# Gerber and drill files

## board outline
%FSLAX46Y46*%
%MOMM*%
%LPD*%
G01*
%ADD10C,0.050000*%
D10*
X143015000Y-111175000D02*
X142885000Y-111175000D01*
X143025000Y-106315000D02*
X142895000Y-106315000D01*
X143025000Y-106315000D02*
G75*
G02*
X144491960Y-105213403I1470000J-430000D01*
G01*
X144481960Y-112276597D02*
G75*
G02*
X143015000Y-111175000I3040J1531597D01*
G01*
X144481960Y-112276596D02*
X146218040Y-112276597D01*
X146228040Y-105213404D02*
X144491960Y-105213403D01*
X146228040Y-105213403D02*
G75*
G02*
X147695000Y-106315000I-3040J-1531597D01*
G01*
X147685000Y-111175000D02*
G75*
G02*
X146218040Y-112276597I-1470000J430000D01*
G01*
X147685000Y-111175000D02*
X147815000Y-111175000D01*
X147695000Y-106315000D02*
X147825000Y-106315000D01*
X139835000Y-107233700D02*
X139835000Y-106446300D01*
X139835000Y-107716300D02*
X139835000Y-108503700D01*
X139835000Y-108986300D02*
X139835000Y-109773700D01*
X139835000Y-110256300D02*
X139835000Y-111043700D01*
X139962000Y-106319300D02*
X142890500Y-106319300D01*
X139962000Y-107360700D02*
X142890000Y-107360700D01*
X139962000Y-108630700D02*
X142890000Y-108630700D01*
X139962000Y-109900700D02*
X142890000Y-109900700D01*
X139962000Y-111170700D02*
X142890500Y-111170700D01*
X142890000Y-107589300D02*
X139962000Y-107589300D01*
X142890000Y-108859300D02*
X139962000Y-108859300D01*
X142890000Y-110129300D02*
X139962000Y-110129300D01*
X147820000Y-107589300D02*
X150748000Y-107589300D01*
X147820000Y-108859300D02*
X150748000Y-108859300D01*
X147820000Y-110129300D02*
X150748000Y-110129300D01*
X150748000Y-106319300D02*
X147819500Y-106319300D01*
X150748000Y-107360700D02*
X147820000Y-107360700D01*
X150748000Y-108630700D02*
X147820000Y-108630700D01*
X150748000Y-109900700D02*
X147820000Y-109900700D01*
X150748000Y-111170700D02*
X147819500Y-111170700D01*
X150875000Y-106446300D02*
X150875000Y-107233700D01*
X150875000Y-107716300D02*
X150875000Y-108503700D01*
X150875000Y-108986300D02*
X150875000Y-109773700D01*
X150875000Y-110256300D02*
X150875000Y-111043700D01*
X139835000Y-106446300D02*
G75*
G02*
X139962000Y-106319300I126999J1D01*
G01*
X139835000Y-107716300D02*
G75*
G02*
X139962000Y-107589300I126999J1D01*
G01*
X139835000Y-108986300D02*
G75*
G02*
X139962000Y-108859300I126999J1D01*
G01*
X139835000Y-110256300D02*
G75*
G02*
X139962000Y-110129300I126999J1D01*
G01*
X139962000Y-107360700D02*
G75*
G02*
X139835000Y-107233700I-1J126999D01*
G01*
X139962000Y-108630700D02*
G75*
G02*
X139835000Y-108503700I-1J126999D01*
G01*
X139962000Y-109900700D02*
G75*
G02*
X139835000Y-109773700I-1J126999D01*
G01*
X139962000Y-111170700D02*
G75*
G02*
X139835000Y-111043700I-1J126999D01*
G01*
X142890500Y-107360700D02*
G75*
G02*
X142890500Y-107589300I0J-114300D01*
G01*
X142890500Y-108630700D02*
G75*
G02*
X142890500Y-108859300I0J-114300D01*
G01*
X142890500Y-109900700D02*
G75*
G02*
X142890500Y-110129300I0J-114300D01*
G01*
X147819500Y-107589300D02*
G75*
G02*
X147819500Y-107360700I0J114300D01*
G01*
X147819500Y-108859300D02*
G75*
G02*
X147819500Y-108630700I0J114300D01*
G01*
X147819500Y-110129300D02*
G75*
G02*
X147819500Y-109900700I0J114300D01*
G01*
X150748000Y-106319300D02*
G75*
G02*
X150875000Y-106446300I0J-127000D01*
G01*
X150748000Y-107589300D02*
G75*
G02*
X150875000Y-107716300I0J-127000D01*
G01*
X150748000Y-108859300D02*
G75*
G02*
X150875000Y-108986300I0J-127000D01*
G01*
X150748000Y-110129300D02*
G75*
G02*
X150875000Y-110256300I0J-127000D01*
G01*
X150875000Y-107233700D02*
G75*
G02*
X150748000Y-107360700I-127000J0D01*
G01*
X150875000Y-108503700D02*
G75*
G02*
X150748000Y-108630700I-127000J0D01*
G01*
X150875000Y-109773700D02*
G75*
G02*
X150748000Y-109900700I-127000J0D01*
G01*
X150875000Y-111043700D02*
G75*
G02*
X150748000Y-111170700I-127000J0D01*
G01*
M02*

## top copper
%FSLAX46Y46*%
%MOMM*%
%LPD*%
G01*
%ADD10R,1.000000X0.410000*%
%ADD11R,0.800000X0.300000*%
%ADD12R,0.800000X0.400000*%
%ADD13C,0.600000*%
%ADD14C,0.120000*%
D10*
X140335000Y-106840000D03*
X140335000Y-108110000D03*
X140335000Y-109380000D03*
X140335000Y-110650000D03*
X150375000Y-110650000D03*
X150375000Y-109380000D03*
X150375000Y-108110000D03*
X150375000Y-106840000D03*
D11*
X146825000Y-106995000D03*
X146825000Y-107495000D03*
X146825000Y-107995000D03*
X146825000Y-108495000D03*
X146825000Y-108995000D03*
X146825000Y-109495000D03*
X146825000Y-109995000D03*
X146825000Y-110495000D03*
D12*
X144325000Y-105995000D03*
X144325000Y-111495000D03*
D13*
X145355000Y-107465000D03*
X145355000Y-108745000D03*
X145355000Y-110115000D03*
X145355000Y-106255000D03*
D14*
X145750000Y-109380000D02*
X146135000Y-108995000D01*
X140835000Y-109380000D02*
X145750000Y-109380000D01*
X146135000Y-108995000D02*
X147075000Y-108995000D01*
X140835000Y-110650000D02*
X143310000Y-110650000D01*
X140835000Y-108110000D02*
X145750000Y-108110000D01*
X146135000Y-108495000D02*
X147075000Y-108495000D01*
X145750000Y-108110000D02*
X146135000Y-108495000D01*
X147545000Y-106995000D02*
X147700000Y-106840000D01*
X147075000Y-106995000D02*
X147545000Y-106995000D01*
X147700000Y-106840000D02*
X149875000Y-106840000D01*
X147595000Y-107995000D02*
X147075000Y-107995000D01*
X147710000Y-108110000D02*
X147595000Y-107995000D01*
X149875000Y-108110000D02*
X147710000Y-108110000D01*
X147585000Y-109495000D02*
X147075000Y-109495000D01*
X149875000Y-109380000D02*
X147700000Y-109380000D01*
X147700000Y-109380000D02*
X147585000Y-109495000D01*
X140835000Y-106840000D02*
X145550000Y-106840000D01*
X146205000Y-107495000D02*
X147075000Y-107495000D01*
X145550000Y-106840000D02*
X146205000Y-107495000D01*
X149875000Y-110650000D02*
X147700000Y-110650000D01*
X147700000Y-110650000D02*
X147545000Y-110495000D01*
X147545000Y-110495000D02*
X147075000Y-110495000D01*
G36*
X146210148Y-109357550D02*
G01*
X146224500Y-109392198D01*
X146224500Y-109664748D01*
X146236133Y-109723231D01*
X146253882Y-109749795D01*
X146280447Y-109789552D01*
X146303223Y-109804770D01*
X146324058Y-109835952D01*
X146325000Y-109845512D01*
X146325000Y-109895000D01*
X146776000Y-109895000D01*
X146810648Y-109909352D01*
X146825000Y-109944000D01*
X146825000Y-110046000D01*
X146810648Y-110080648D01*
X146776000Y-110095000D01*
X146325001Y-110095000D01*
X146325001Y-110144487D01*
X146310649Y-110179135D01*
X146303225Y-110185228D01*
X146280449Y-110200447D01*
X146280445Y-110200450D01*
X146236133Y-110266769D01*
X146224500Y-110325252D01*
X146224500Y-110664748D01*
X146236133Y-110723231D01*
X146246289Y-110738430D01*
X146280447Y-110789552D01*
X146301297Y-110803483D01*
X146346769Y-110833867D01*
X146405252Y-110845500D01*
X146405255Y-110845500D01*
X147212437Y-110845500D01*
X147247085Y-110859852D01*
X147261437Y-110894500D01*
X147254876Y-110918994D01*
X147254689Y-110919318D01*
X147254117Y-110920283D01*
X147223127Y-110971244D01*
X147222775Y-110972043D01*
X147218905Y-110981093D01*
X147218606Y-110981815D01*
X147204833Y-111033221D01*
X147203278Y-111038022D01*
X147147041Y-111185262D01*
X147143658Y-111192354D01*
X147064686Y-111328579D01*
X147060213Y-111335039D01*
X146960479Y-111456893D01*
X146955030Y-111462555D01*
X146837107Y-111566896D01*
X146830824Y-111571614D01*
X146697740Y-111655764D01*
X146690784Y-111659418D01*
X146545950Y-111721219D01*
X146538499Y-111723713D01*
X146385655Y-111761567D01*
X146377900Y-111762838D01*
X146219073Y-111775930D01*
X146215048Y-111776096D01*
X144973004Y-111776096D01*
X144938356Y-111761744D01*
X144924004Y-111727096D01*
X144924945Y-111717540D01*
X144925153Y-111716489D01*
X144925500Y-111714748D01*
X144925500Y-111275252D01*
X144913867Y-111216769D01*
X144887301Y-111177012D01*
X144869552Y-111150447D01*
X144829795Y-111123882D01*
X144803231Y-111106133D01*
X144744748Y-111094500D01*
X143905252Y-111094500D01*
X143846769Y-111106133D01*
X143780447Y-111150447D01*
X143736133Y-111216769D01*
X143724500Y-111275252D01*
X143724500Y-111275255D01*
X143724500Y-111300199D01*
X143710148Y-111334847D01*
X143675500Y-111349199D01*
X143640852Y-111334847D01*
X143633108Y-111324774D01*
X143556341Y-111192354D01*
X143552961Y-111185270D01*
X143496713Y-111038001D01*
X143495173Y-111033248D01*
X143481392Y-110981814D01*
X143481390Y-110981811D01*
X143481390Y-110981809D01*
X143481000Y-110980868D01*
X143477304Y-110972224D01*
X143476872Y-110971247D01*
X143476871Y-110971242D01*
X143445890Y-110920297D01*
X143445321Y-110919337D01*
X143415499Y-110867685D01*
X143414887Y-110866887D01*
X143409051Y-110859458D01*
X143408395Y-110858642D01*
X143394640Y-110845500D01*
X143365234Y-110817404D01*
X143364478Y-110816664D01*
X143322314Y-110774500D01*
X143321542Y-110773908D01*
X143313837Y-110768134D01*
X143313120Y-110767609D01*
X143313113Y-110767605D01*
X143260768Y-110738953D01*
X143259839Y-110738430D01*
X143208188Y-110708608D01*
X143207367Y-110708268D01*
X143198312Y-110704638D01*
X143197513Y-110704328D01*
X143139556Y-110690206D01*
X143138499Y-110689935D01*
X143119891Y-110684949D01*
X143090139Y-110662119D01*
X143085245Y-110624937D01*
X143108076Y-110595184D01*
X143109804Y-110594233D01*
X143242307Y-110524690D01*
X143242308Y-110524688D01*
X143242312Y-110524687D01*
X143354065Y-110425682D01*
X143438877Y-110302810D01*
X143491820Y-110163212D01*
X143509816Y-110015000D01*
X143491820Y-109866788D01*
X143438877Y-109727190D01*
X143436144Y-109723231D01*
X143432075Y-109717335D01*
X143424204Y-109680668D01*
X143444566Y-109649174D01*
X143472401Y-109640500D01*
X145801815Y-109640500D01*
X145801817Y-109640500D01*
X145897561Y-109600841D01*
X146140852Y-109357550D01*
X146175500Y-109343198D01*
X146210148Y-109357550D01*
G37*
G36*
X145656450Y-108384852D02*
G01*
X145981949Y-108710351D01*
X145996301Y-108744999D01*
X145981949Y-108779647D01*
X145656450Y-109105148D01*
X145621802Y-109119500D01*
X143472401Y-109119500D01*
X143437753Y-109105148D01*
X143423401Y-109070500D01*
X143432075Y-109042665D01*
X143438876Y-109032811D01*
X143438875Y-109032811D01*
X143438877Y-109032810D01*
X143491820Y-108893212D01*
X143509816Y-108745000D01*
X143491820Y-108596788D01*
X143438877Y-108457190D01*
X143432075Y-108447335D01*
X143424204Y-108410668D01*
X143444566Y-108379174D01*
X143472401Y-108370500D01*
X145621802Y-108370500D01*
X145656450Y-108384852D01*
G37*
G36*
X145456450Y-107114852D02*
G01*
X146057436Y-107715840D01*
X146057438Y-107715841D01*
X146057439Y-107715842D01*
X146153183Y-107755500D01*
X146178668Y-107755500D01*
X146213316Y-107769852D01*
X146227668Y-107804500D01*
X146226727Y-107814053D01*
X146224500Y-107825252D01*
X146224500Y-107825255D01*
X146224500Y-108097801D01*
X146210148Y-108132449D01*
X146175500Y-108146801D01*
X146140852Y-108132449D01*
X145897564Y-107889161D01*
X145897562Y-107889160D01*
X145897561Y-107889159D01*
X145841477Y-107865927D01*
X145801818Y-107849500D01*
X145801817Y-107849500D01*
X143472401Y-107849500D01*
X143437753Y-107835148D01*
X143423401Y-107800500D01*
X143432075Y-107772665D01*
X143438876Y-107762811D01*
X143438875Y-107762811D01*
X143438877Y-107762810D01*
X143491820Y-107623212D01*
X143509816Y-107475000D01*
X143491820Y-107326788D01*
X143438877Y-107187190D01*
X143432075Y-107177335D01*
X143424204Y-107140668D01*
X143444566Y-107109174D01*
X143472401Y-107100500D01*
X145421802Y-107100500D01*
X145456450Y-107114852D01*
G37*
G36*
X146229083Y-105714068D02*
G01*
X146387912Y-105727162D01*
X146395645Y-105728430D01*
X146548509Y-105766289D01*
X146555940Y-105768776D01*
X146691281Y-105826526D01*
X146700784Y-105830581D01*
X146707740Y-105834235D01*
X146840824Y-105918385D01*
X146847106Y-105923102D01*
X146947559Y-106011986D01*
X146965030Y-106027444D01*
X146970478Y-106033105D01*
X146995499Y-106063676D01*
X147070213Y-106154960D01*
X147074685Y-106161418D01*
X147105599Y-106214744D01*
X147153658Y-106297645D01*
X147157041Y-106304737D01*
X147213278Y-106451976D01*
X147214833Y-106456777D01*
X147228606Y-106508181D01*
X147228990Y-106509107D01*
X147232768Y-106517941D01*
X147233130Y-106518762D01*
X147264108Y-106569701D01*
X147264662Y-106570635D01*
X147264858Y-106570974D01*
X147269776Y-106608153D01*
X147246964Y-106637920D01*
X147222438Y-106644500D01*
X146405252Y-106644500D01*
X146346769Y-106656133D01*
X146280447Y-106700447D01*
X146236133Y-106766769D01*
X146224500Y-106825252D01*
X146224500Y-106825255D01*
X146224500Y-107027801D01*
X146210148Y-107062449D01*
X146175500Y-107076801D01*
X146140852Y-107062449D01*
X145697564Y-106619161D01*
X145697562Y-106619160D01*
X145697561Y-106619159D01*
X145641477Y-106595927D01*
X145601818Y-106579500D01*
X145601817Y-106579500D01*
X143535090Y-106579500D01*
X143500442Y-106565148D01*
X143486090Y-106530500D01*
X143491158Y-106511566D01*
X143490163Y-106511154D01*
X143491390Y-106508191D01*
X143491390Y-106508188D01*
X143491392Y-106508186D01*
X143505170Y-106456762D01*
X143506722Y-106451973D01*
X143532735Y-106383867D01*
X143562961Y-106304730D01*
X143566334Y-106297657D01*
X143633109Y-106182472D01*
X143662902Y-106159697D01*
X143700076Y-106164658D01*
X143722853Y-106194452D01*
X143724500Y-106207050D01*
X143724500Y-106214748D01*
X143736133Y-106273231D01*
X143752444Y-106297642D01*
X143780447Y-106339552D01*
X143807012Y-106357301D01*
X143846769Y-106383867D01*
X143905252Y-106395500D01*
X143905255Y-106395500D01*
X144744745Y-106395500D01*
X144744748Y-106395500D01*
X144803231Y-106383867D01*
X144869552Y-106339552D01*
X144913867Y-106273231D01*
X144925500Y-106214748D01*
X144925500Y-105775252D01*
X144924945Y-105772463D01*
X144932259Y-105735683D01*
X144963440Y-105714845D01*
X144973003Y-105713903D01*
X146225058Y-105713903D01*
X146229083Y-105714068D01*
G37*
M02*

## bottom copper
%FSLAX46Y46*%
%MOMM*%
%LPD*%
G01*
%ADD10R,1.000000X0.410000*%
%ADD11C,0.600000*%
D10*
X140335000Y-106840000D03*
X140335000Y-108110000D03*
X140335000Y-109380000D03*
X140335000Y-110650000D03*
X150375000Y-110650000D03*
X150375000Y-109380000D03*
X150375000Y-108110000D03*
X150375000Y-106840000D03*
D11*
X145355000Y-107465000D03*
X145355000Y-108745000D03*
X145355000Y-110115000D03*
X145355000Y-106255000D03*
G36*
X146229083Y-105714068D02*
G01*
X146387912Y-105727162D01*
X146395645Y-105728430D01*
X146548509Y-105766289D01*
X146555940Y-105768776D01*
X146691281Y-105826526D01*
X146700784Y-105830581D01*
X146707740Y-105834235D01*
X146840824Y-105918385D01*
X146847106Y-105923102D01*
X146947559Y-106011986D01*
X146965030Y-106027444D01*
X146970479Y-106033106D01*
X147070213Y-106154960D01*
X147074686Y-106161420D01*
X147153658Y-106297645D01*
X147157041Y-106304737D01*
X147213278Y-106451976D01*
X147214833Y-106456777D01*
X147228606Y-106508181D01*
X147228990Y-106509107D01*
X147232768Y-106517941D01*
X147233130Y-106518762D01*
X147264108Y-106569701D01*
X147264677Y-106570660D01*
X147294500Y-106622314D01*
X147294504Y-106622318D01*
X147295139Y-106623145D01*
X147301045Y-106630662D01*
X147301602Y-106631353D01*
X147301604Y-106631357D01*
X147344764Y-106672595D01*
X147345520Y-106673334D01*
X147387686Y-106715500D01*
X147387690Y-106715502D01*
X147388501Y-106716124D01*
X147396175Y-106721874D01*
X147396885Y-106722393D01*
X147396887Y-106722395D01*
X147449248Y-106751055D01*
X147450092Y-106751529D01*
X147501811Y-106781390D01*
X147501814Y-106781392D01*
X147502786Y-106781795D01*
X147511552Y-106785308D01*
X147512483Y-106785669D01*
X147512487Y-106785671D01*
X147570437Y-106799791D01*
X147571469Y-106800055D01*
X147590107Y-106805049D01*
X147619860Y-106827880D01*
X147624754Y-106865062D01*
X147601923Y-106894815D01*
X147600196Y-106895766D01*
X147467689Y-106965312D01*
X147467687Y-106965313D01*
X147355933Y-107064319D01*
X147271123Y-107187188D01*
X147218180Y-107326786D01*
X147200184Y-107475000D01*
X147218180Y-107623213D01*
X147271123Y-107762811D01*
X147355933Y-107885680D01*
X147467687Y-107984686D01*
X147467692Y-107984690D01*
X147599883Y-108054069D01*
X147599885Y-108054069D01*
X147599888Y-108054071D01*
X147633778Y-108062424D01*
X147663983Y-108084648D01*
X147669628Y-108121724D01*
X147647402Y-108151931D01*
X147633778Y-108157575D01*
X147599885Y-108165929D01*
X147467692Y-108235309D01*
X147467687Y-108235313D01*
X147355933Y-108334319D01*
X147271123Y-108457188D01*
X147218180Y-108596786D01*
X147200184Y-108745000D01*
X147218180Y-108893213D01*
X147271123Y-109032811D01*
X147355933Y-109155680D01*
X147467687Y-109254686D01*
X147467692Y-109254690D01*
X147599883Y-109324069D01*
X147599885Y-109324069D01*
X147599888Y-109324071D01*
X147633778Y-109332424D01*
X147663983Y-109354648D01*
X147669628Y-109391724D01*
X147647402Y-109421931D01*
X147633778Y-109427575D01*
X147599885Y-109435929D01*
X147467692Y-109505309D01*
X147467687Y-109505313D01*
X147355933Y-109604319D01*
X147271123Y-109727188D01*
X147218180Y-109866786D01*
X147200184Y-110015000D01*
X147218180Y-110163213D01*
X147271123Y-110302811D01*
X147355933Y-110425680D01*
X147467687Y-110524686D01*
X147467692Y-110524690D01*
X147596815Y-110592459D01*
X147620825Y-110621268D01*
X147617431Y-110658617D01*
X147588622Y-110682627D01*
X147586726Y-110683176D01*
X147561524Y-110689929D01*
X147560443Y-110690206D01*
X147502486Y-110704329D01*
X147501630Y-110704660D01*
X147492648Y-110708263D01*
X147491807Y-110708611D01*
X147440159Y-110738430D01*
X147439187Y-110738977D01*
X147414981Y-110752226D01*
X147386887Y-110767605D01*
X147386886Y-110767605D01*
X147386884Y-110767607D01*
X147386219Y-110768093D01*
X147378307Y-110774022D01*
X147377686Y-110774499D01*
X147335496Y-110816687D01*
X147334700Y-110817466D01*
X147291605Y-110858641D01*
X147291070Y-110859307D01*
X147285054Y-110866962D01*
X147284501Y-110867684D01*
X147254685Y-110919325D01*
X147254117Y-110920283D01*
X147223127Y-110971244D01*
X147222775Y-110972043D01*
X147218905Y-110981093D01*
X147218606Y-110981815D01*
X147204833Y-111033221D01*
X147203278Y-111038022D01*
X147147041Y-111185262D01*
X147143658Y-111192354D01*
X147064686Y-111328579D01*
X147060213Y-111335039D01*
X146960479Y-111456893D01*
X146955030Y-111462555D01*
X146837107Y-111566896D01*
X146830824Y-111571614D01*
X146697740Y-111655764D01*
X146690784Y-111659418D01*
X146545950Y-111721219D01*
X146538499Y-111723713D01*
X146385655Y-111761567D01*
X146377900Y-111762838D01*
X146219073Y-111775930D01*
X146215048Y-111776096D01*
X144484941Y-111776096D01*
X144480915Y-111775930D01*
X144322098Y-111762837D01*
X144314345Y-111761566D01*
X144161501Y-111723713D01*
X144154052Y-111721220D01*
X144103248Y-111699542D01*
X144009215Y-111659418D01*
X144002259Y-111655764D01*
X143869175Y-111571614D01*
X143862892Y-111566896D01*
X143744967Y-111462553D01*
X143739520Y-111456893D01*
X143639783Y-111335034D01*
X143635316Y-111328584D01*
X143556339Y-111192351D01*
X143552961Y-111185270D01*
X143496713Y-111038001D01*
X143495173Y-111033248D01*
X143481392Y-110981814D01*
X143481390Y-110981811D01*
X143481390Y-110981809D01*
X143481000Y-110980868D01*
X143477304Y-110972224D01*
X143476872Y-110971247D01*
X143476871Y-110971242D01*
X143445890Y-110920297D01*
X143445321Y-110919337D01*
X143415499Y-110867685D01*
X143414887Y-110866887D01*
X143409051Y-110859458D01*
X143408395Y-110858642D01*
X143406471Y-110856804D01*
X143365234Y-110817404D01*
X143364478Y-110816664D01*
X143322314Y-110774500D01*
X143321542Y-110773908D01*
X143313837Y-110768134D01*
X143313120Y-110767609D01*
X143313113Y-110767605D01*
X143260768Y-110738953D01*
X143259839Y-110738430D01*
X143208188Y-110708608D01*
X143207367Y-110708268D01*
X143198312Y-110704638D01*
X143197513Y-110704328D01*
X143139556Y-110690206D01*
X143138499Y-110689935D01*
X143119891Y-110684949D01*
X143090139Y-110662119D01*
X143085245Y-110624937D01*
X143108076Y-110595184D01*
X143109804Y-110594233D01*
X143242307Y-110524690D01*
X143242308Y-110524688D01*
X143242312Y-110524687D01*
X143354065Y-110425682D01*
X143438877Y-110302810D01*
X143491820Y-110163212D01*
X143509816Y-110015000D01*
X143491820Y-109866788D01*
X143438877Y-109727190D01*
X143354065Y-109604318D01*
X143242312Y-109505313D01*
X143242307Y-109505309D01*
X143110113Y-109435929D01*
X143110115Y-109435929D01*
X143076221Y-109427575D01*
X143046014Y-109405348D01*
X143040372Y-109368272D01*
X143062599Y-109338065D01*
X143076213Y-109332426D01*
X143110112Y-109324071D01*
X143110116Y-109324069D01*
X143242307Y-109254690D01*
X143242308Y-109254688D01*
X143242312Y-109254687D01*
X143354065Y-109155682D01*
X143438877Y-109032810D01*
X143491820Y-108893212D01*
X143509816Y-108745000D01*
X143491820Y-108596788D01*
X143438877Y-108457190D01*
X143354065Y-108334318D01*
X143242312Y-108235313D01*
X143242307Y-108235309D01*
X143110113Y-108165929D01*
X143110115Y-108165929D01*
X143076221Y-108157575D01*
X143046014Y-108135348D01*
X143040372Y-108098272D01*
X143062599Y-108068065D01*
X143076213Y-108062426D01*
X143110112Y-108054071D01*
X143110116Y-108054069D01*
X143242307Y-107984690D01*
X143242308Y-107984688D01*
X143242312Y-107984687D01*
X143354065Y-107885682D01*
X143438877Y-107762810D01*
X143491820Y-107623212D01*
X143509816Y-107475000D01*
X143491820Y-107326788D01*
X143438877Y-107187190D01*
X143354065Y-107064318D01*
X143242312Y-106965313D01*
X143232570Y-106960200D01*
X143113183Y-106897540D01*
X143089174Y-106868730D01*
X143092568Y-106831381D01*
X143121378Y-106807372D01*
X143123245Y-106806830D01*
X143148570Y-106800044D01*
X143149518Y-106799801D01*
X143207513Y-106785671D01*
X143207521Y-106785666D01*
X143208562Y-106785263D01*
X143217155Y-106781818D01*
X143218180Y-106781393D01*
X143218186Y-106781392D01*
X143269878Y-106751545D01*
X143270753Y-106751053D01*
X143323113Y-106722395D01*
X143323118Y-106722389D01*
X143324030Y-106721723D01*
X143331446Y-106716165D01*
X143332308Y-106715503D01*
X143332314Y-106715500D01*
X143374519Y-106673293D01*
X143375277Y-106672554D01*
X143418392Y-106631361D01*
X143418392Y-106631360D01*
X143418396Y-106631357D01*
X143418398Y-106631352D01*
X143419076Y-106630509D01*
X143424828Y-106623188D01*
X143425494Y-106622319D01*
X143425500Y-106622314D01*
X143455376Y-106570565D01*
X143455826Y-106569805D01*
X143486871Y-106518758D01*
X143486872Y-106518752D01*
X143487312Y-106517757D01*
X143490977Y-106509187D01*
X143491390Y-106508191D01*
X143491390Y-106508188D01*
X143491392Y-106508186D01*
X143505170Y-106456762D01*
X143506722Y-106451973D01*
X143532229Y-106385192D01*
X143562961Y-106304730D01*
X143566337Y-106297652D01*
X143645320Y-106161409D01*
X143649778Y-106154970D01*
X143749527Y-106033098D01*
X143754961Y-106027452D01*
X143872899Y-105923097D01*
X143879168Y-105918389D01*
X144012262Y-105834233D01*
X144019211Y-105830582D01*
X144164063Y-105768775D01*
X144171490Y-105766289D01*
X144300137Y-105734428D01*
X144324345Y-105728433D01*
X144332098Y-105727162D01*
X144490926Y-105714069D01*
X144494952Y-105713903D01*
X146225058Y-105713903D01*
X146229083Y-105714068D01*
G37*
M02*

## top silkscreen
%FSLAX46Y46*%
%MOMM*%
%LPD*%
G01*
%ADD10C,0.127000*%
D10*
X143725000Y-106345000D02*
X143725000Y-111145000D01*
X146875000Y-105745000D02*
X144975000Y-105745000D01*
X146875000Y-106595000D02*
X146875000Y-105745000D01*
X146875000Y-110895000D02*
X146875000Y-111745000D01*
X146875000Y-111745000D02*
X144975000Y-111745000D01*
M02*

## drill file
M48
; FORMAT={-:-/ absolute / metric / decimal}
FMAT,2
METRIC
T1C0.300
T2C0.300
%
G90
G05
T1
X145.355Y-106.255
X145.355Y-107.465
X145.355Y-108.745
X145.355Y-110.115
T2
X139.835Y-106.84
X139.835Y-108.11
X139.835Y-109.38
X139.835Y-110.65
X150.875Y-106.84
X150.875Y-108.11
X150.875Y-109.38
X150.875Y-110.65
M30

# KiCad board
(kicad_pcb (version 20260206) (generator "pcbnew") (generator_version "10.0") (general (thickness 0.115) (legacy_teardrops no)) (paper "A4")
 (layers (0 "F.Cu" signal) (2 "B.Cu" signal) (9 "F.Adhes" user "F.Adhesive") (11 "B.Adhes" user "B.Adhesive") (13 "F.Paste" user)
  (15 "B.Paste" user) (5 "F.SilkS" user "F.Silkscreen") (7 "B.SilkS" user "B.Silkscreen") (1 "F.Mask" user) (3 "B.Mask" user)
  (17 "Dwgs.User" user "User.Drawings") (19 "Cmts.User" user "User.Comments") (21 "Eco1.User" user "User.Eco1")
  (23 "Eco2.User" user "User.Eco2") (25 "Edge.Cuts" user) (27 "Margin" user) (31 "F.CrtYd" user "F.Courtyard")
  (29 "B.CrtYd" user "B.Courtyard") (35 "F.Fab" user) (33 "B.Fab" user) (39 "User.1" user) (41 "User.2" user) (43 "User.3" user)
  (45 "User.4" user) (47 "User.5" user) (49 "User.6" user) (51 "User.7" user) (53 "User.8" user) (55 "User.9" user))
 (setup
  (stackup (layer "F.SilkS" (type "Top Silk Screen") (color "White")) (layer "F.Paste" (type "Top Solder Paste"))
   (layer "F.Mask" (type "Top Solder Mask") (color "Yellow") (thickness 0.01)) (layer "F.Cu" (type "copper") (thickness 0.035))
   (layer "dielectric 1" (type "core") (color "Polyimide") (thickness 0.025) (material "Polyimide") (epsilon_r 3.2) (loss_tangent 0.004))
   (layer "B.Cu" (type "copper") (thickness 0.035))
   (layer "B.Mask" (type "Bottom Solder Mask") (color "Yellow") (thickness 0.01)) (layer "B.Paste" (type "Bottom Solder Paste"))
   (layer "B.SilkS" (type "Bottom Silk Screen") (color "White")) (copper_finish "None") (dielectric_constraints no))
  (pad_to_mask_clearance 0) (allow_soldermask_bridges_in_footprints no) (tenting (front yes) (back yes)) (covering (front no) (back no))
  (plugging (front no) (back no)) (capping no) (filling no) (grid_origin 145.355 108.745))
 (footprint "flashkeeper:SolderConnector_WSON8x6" (layer "F.Cu") (at 145.355 108.745)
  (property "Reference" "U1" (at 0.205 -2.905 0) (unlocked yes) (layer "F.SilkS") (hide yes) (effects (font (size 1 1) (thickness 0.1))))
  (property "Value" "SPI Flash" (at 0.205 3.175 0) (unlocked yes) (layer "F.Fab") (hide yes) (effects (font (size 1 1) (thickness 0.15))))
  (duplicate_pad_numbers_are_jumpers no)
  (fp_line (start -5.52 -1.5113) (end -5.52 -2.2987) (stroke (width 0.05) (type default)) (layer "Edge.Cuts"))
  (fp_line (start -5.52 -1.0287) (end -5.52 -0.2413) (stroke (width 0.05) (type default)) (layer "Edge.Cuts"))
  (fp_line (start -5.52 0.2413) (end -5.52 1.0287) (stroke (width 0.05) (type default)) (layer "Edge.Cuts"))
  (fp_line (start -5.52 1.5113) (end -5.52 2.2987) (stroke (width 0.05) (type default)) (layer "Edge.Cuts"))
  (fp_line (start -5.393 -2.4257) (end -2.4645 -2.4257) (stroke (width 0.05) (type default)) (layer "Edge.Cuts"))
  (fp_line (start -5.393 -1.3843) (end -2.465 -1.3843) (stroke (width 0.05) (type default)) (layer "Edge.Cuts"))
  (fp_line (start -5.393 -0.1143) (end -2.465 -0.1143) (stroke (width 0.05) (type default)) (layer "Edge.Cuts"))
  (fp_line (start -5.393 1.1557) (end -2.465 1.1557) (stroke (width 0.05) (type default)) (layer "Edge.Cuts"))
  (fp_line (start -5.393 2.4257) (end -2.4645 2.4257) (stroke (width 0.05) (type default)) (layer "Edge.Cuts"))
  (fp_line (start -2.465 -1.1557) (end -5.393 -1.1557) (stroke (width 0.05) (type default)) (layer "Edge.Cuts"))
  (fp_line (start -2.465 0.1143) (end -5.393 0.1143) (stroke (width 0.05) (type default)) (layer "Edge.Cuts"))
  (fp_line (start -2.465 1.3843) (end -5.393 1.3843) (stroke (width 0.05) (type default)) (layer "Edge.Cuts"))
  (fp_line (start 2.465 -1.1557) (end 5.393 -1.1557) (stroke (width 0.05) (type default)) (layer "Edge.Cuts"))
  (fp_line (start 2.465 0.1143) (end 5.393 0.1143) (stroke (width 0.05) (type default)) (layer "Edge.Cuts"))
  (fp_line (start 2.465 1.3843) (end 5.393 1.3843) (stroke (width 0.05) (type default)) (layer "Edge.Cuts"))
  (fp_line (start 5.393 -2.4257) (end 2.4645 -2.4257) (stroke (width 0.05) (type default)) (layer "Edge.Cuts"))
  (fp_line (start 5.393 -1.3843) (end 2.465 -1.3843) (stroke (width 0.05) (type default)) (layer "Edge.Cuts"))
  (fp_line (start 5.393 -0.1143) (end 2.465 -0.1143) (stroke (width 0.05) (type default)) (layer "Edge.Cuts"))
  (fp_line (start 5.393 1.1557) (end 2.465 1.1557) (stroke (width 0.05) (type default)) (layer "Edge.Cuts"))
  (fp_line (start 5.393 2.4257) (end 2.4645 2.4257) (stroke (width 0.05) (type default)) (layer "Edge.Cuts"))
  (fp_line (start 5.52 -2.2987) (end 5.52 -1.5113) (stroke (width 0.05) (type default)) (layer "Edge.Cuts"))
  (fp_line (start 5.52 -1.0287) (end 5.52 -0.2413) (stroke (width 0.05) (type default)) (layer "Edge.Cuts"))
  (fp_line (start 5.52 0.2413) (end 5.52 1.0287) (stroke (width 0.05) (type default)) (layer "Edge.Cuts"))
  (fp_line (start 5.52 1.5113) (end 5.52 2.2987) (stroke (width 0.05) (type default)) (layer "Edge.Cuts"))
  (fp_arc (start -5.52 -2.2987) (mid -5.482803 -2.388503) (end -5.393 -2.4257) (stroke (width 0.05) (type default)) (layer "Edge.Cuts"))
  (fp_arc (start -5.52 -1.0287) (mid -5.482803 -1.118503) (end -5.393 -1.1557) (stroke (width 0.05) (type default)) (layer "Edge.Cuts"))
  (fp_arc (start -5.52 0.2413) (mid -5.482803 0.151497) (end -5.393 0.1143) (stroke (width 0.05) (type default)) (layer "Edge.Cuts"))
  (fp_arc (start -5.52 1.5113) (mid -5.482803 1.421497) (end -5.393 1.3843) (stroke (width 0.05) (type default)) (layer "Edge.Cuts"))
  (fp_arc (start -5.393 -1.3843) (mid -5.482803 -1.421497) (end -5.52 -1.5113) (stroke (width 0.05) (type default)) (layer "Edge.Cuts"))
  (fp_arc (start -5.393 -0.1143) (mid -5.482803 -0.151497) (end -5.52 -0.2413) (stroke (width 0.05) (type default)) (layer "Edge.Cuts"))
  (fp_arc (start -5.393 1.1557) (mid -5.482803 1.118503) (end -5.52 1.0287) (stroke (width 0.05) (type default)) (layer "Edge.Cuts"))
  (fp_arc (start -5.393 2.4257) (mid -5.482803 2.388503) (end -5.52 2.2987) (stroke (width 0.05) (type default)) (layer "Edge.Cuts"))
  (fp_arc (start -2.4645 -1.3843) (mid -2.3502 -1.27) (end -2.4645 -1.1557) (stroke (width 0.05) (type default)) (layer "Edge.Cuts"))
  (fp_arc (start -2.4645 -0.1143) (mid -2.3502 0) (end -2.4645 0.1143) (stroke (width 0.05) (type default)) (layer "Edge.Cuts"))
  (fp_arc (start -2.4645 1.1557) (mid -2.3502 1.27) (end -2.4645 1.3843) (stroke (width 0.05) (type default)) (layer "Edge.Cuts"))
  (fp_arc (start 2.4645 -1.1557) (mid 2.3502 -1.27) (end 2.4645 -1.3843) (stroke (width 0.05) (type default)) (layer "Edge.Cuts"))
  (fp_arc (start 2.4645 0.1143) (mid 2.3502 0) (end 2.4645 -0.1143) (stroke (width 0.05) (type default)) (layer "Edge.Cuts"))
  (fp_arc (start 2.4645 1.3843) (mid 2.3502 1.27) (end 2.4645 1.1557) (stroke (width 0.05) (type default)) (layer "Edge.Cuts"))
  (fp_arc (start 5.393 -2.4257) (mid 5.482803 -2.388503) (end 5.52 -2.2987) (stroke (width 0.05) (type default)) (layer "Edge.Cuts"))
  (fp_arc (start 5.393 -1.1557) (mid 5.482803 -1.118503) (end 5.52 -1.0287) (stroke (width 0.05) (type default)) (layer "Edge.Cuts"))
  (fp_arc (start 5.393 0.1143) (mid 5.482803 0.151497) (end 5.52 0.2413) (stroke (width 0.05) (type default)) (layer "Edge.Cuts"))
  (fp_arc (start 5.393 1.3843) (mid 5.482803 1.421497) (end 5.52 1.5113) (stroke (width 0.05) (type default)) (layer "Edge.Cuts"))
  (fp_arc (start 5.52 -1.5113) (mid 5.482803 -1.421497) (end 5.393 -1.3843) (stroke (width 0.05) (type default)) (layer "Edge.Cuts"))
  (fp_arc (start 5.52 -0.2413) (mid 5.482803 -0.151497) (end 5.393 -0.1143) (stroke (width 0.05) (type default)) (layer "Edge.Cuts"))
  (fp_arc (start 5.52 1.0287) (mid 5.482803 1.118503) (end 5.393 1.1557) (stroke (width 0.05) (type default)) (layer "Edge.Cuts"))
  (fp_arc (start 5.52 2.2987) (mid 5.482803 2.388503) (end 5.393 2.4257) (stroke (width 0.05) (type default)) (layer "Edge.Cuts"))
  (pad "1" thru_hole rect (at -5.52 -1.905) (size 1 0.41) (drill 0.3 (offset 0.5 0)) (layers "*.Cu" "*.Mask") (remove_unused_layers no)
   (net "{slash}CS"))
  (pad "2" thru_hole rect (at -5.52 -0.635) (size 1 0.41) (drill 0.3 (offset 0.5 0)) (layers "*.Cu" "*.Mask") (remove_unused_layers no)
   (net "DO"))
  (pad "3" thru_hole rect (at -5.52 0.635) (size 1 0.41) (drill 0.3 (offset 0.5 0)) (layers "*.Cu" "*.Mask") (remove_unused_layers no)
   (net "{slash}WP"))
  (pad "4" thru_hole rect (at -5.52 1.905) (size 1 0.41) (drill 0.3 (offset 0.5 0)) (layers "*.Cu" "*.Mask") (remove_unused_layers no)
   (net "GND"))
  (pad "5" thru_hole rect (at 5.52 1.905 180) (size 1 0.41) (drill 0.3 (offset 0.5 0)) (layers "*.Cu" "*.Mask") (remove_unused_layers no)
   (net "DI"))
  (pad "6" thru_hole rect (at 5.52 0.635 180) (size 1 0.41) (drill 0.3 (offset 0.5 0)) (layers "*.Cu" "*.Mask") (remove_unused_layers no)
   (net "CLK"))
  (pad "7" thru_hole rect (at 5.52 -0.635 180) (size 1 0.41) (drill 0.3 (offset 0.5 0)) (layers "*.Cu" "*.Mask") (remove_unused_layers no)
   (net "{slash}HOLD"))
  (pad "8" thru_hole rect (at 5.52 -1.905 180) (size 1 0.41) (drill 0.3 (offset 0.5 0)) (layers "*.Cu" "*.Mask") (remove_unused_layers no)
   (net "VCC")))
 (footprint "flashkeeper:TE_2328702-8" (layer "F.Cu") (at 146.825 110.495 -90)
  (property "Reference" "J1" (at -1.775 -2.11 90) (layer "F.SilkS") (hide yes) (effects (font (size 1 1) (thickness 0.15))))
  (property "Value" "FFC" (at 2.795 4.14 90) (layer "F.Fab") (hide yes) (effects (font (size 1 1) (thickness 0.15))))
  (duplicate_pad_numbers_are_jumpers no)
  (fp_line (start -4.15 3.1) (end 0.65 3.1) (stroke (width 0.127) (type solid)) (layer "F.SilkS"))
  (fp_line (start -4.75 -0.05) (end -4.75 1.85) (stroke (width 0.127) (type solid)) (layer "F.SilkS"))
  (fp_line (start -3.9 -0.05) (end -4.75 -0.05) (stroke (width 0.127) (type solid)) (layer "F.SilkS"))
  (fp_line (start 0.4 -0.05) (end 1.25 -0.05) (stroke (width 0.127) (type solid)) (layer "F.SilkS"))
  (fp_line (start 1.25 -0.05) (end 1.25 1.85) (stroke (width 0.127) (type solid)) (layer "F.SilkS"))
  (pad "1" smd rect (at -3.5 0 270) (size 0.3 0.8) (layers "F.Cu" "F.Mask" "F.Paste") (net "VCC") (solder_mask_margin 0.102))
  (pad "2" smd rect (at -3 0 270) (size 0.3 0.8) (layers "F.Cu" "F.Mask" "F.Paste") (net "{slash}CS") (solder_mask_margin 0.102))
  (pad "3" smd rect (at -2.5 0 270) (size 0.3 0.8) (layers "F.Cu" "F.Mask" "F.Paste") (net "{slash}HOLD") (solder_mask_margin 0.102))
  (pad "4" smd rect (at -2 0 270) (size 0.3 0.8) (layers "F.Cu" "F.Mask" "F.Paste") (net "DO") (solder_mask_margin 0.102))
  (pad "5" smd rect (at -1.5 0 270) (size 0.3 0.8) (layers "F.Cu" "F.Mask" "F.Paste") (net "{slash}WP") (solder_mask_margin 0.102))
  (pad "6" smd rect (at -1 0 270) (size 0.3 0.8) (layers "F.Cu" "F.Mask" "F.Paste") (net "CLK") (solder_mask_margin 0.102))
  (pad "7" smd rect (at -0.5 0 270) (size 0.3 0.8) (layers "F.Cu" "F.Mask" "F.Paste") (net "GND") (solder_mask_margin 0.102))
  (pad "8" smd rect (at 0 0 270) (size 0.3 0.8) (layers "F.Cu" "F.Mask" "F.Paste") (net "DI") (solder_mask_margin 0.102))
  (pad "S1" smd rect (at -4.5 2.5 270) (size 0.4 0.8) (layers "F.Cu" "F.Mask" "F.Paste") (solder_mask_margin 0.102))
  (pad "S2" smd rect (at 1 2.5 270) (size 0.4 0.8) (layers "F.Cu" "F.Mask" "F.Paste") (solder_mask_margin 0.102)))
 (gr_line (start 143.015 111.175) (end 142.885 111.175) (stroke (width 0.05) (type default)) (layer "Edge.Cuts"))
 (gr_line (start 143.025 106.315) (end 142.895 106.315) (stroke (width 0.05) (type default)) (layer "Edge.Cuts"))
 (gr_arc (start 143.025 106.315) (mid 143.575304 105.520272) (end 144.49196 105.213403) (stroke (width 0.05) (type default))
  (layer "Edge.Cuts"))
 (gr_arc (start 144.48196 112.276597) (mid 143.565304 111.969728) (end 143.015 111.175) (stroke (width 0.05) (type default))
  (layer "Edge.Cuts"))
 (gr_line (start 144.48196 112.276596) (end 146.21804 112.276597) (stroke (width 0.05) (type default)) (layer "Edge.Cuts"))
 (gr_line (start 146.22804 105.213404) (end 144.49196 105.213403) (stroke (width 0.05) (type default)) (layer "Edge.Cuts"))
 (gr_arc (start 146.22804 105.213403) (mid 147.144696 105.520272) (end 147.695 106.315) (stroke (width 0.05) (type default))
  (layer "Edge.Cuts"))
 (gr_arc (start 147.685 111.175) (mid 147.134696 111.969728) (end 146.21804 112.276597) (stroke (width 0.05) (type default))
  (layer "Edge.Cuts"))
 (gr_line (start 147.685 111.175) (end 147.815 111.175) (stroke (width 0.05) (type default)) (layer "Edge.Cuts"))
 (gr_line (start 147.695 106.315) (end 147.825 106.315) (stroke (width 0.05) (type default)) (layer "Edge.Cuts"))
 (segment (start 145.75 109.38) (end 146.135 108.995) (width 0.12) (layer "F.Cu") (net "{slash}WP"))
 (segment (start 140.835 109.38) (end 145.75 109.38) (width 0.12) (layer "F.Cu") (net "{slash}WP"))
 (segment (start 146.135 108.995) (end 147.075 108.995) (width 0.12) (layer "F.Cu") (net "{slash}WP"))
 (segment (start 140.835 110.65) (end 143.31 110.65) (width 0.12) (layer "F.Cu") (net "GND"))
 (via (at 145.355 107.465) (size 0.6) (drill 0.3) (layers "F.Cu" "B.Cu") (free yes) (capping no) (covering (front no) (back no))
  (plugging (front no) (back no)) (filling no) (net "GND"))
 (via (at 145.355 108.745) (size 0.6) (drill 0.3) (layers "F.Cu" "B.Cu") (free yes) (capping no) (covering (front no) (back no))
  (plugging (front no) (back no)) (filling no) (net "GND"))
 (via (at 145.355 110.115) (size 0.6) (drill 0.3) (layers "F.Cu" "B.Cu") (free yes) (capping no) (covering (front no) (back no))
  (plugging (front no) (back no)) (filling no) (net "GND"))
 (via (at 145.355 106.255) (size 0.6) (drill 0.3) (layers "F.Cu" "B.Cu") (free yes) (capping no) (covering (front no) (back no))
  (plugging (front no) (back no)) (filling no) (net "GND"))
 (segment (start 140.835 108.11) (end 145.75 108.11) (width 0.12) (layer "F.Cu") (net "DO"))
 (segment (start 146.135 108.495) (end 147.075 108.495) (width 0.12) (layer "F.Cu") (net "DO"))
 (segment (start 145.75 108.11) (end 146.135 108.495) (width 0.12) (layer "F.Cu") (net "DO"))
 (segment (start 147.545 106.995) (end 147.7 106.84) (width 0.12) (layer "F.Cu") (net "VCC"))
 (segment (start 147.075 106.995) (end 147.545 106.995) (width 0.12) (layer "F.Cu") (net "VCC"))
 (segment (start 147.7 106.84) (end 149.875 106.84) (width 0.12) (layer "F.Cu") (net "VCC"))
 (segment (start 147.595 107.995) (end 147.075 107.995) (width 0.12) (layer "F.Cu") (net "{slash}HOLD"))
 (segment (start 147.71 108.11) (end 147.595 107.995) (width 0.12) (layer "F.Cu") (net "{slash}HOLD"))
 (segment (start 149.875 108.11) (end 147.71 108.11) (width 0.12) (layer "F.Cu") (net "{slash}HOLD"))
 (segment (start 147.585 109.495) (end 147.075 109.495) (width 0.12) (layer "F.Cu") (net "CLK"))
 (segment (start 149.875 109.38) (end 147.7 109.38) (width 0.12) (layer "F.Cu") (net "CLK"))
 (segment (start 147.7 109.38) (end 147.585 109.495) (width 0.12) (layer "F.Cu") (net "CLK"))
 (segment (start 140.835 106.84) (end 145.55 106.84) (width 0.12) (layer "F.Cu") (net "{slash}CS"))
 (segment (start 146.205 107.495) (end 147.075 107.495) (width 0.12) (layer "F.Cu") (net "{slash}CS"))
 (segment (start 145.55 106.84) (end 146.205 107.495) (width 0.12) (layer "F.Cu") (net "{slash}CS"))
 (segment (start 149.875 110.65) (end 147.7 110.65) (width 0.12) (layer "F.Cu") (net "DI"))
 (segment (start 147.7 110.65) (end 147.545 110.495) (width 0.12) (layer "F.Cu") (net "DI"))
 (segment (start 147.545 110.495) (end 147.075 110.495) (width 0.12) (layer "F.Cu") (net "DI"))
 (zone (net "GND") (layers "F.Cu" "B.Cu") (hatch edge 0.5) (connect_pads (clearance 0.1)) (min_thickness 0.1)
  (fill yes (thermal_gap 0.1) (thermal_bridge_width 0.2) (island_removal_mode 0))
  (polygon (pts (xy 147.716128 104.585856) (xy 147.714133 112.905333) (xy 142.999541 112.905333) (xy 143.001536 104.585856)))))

